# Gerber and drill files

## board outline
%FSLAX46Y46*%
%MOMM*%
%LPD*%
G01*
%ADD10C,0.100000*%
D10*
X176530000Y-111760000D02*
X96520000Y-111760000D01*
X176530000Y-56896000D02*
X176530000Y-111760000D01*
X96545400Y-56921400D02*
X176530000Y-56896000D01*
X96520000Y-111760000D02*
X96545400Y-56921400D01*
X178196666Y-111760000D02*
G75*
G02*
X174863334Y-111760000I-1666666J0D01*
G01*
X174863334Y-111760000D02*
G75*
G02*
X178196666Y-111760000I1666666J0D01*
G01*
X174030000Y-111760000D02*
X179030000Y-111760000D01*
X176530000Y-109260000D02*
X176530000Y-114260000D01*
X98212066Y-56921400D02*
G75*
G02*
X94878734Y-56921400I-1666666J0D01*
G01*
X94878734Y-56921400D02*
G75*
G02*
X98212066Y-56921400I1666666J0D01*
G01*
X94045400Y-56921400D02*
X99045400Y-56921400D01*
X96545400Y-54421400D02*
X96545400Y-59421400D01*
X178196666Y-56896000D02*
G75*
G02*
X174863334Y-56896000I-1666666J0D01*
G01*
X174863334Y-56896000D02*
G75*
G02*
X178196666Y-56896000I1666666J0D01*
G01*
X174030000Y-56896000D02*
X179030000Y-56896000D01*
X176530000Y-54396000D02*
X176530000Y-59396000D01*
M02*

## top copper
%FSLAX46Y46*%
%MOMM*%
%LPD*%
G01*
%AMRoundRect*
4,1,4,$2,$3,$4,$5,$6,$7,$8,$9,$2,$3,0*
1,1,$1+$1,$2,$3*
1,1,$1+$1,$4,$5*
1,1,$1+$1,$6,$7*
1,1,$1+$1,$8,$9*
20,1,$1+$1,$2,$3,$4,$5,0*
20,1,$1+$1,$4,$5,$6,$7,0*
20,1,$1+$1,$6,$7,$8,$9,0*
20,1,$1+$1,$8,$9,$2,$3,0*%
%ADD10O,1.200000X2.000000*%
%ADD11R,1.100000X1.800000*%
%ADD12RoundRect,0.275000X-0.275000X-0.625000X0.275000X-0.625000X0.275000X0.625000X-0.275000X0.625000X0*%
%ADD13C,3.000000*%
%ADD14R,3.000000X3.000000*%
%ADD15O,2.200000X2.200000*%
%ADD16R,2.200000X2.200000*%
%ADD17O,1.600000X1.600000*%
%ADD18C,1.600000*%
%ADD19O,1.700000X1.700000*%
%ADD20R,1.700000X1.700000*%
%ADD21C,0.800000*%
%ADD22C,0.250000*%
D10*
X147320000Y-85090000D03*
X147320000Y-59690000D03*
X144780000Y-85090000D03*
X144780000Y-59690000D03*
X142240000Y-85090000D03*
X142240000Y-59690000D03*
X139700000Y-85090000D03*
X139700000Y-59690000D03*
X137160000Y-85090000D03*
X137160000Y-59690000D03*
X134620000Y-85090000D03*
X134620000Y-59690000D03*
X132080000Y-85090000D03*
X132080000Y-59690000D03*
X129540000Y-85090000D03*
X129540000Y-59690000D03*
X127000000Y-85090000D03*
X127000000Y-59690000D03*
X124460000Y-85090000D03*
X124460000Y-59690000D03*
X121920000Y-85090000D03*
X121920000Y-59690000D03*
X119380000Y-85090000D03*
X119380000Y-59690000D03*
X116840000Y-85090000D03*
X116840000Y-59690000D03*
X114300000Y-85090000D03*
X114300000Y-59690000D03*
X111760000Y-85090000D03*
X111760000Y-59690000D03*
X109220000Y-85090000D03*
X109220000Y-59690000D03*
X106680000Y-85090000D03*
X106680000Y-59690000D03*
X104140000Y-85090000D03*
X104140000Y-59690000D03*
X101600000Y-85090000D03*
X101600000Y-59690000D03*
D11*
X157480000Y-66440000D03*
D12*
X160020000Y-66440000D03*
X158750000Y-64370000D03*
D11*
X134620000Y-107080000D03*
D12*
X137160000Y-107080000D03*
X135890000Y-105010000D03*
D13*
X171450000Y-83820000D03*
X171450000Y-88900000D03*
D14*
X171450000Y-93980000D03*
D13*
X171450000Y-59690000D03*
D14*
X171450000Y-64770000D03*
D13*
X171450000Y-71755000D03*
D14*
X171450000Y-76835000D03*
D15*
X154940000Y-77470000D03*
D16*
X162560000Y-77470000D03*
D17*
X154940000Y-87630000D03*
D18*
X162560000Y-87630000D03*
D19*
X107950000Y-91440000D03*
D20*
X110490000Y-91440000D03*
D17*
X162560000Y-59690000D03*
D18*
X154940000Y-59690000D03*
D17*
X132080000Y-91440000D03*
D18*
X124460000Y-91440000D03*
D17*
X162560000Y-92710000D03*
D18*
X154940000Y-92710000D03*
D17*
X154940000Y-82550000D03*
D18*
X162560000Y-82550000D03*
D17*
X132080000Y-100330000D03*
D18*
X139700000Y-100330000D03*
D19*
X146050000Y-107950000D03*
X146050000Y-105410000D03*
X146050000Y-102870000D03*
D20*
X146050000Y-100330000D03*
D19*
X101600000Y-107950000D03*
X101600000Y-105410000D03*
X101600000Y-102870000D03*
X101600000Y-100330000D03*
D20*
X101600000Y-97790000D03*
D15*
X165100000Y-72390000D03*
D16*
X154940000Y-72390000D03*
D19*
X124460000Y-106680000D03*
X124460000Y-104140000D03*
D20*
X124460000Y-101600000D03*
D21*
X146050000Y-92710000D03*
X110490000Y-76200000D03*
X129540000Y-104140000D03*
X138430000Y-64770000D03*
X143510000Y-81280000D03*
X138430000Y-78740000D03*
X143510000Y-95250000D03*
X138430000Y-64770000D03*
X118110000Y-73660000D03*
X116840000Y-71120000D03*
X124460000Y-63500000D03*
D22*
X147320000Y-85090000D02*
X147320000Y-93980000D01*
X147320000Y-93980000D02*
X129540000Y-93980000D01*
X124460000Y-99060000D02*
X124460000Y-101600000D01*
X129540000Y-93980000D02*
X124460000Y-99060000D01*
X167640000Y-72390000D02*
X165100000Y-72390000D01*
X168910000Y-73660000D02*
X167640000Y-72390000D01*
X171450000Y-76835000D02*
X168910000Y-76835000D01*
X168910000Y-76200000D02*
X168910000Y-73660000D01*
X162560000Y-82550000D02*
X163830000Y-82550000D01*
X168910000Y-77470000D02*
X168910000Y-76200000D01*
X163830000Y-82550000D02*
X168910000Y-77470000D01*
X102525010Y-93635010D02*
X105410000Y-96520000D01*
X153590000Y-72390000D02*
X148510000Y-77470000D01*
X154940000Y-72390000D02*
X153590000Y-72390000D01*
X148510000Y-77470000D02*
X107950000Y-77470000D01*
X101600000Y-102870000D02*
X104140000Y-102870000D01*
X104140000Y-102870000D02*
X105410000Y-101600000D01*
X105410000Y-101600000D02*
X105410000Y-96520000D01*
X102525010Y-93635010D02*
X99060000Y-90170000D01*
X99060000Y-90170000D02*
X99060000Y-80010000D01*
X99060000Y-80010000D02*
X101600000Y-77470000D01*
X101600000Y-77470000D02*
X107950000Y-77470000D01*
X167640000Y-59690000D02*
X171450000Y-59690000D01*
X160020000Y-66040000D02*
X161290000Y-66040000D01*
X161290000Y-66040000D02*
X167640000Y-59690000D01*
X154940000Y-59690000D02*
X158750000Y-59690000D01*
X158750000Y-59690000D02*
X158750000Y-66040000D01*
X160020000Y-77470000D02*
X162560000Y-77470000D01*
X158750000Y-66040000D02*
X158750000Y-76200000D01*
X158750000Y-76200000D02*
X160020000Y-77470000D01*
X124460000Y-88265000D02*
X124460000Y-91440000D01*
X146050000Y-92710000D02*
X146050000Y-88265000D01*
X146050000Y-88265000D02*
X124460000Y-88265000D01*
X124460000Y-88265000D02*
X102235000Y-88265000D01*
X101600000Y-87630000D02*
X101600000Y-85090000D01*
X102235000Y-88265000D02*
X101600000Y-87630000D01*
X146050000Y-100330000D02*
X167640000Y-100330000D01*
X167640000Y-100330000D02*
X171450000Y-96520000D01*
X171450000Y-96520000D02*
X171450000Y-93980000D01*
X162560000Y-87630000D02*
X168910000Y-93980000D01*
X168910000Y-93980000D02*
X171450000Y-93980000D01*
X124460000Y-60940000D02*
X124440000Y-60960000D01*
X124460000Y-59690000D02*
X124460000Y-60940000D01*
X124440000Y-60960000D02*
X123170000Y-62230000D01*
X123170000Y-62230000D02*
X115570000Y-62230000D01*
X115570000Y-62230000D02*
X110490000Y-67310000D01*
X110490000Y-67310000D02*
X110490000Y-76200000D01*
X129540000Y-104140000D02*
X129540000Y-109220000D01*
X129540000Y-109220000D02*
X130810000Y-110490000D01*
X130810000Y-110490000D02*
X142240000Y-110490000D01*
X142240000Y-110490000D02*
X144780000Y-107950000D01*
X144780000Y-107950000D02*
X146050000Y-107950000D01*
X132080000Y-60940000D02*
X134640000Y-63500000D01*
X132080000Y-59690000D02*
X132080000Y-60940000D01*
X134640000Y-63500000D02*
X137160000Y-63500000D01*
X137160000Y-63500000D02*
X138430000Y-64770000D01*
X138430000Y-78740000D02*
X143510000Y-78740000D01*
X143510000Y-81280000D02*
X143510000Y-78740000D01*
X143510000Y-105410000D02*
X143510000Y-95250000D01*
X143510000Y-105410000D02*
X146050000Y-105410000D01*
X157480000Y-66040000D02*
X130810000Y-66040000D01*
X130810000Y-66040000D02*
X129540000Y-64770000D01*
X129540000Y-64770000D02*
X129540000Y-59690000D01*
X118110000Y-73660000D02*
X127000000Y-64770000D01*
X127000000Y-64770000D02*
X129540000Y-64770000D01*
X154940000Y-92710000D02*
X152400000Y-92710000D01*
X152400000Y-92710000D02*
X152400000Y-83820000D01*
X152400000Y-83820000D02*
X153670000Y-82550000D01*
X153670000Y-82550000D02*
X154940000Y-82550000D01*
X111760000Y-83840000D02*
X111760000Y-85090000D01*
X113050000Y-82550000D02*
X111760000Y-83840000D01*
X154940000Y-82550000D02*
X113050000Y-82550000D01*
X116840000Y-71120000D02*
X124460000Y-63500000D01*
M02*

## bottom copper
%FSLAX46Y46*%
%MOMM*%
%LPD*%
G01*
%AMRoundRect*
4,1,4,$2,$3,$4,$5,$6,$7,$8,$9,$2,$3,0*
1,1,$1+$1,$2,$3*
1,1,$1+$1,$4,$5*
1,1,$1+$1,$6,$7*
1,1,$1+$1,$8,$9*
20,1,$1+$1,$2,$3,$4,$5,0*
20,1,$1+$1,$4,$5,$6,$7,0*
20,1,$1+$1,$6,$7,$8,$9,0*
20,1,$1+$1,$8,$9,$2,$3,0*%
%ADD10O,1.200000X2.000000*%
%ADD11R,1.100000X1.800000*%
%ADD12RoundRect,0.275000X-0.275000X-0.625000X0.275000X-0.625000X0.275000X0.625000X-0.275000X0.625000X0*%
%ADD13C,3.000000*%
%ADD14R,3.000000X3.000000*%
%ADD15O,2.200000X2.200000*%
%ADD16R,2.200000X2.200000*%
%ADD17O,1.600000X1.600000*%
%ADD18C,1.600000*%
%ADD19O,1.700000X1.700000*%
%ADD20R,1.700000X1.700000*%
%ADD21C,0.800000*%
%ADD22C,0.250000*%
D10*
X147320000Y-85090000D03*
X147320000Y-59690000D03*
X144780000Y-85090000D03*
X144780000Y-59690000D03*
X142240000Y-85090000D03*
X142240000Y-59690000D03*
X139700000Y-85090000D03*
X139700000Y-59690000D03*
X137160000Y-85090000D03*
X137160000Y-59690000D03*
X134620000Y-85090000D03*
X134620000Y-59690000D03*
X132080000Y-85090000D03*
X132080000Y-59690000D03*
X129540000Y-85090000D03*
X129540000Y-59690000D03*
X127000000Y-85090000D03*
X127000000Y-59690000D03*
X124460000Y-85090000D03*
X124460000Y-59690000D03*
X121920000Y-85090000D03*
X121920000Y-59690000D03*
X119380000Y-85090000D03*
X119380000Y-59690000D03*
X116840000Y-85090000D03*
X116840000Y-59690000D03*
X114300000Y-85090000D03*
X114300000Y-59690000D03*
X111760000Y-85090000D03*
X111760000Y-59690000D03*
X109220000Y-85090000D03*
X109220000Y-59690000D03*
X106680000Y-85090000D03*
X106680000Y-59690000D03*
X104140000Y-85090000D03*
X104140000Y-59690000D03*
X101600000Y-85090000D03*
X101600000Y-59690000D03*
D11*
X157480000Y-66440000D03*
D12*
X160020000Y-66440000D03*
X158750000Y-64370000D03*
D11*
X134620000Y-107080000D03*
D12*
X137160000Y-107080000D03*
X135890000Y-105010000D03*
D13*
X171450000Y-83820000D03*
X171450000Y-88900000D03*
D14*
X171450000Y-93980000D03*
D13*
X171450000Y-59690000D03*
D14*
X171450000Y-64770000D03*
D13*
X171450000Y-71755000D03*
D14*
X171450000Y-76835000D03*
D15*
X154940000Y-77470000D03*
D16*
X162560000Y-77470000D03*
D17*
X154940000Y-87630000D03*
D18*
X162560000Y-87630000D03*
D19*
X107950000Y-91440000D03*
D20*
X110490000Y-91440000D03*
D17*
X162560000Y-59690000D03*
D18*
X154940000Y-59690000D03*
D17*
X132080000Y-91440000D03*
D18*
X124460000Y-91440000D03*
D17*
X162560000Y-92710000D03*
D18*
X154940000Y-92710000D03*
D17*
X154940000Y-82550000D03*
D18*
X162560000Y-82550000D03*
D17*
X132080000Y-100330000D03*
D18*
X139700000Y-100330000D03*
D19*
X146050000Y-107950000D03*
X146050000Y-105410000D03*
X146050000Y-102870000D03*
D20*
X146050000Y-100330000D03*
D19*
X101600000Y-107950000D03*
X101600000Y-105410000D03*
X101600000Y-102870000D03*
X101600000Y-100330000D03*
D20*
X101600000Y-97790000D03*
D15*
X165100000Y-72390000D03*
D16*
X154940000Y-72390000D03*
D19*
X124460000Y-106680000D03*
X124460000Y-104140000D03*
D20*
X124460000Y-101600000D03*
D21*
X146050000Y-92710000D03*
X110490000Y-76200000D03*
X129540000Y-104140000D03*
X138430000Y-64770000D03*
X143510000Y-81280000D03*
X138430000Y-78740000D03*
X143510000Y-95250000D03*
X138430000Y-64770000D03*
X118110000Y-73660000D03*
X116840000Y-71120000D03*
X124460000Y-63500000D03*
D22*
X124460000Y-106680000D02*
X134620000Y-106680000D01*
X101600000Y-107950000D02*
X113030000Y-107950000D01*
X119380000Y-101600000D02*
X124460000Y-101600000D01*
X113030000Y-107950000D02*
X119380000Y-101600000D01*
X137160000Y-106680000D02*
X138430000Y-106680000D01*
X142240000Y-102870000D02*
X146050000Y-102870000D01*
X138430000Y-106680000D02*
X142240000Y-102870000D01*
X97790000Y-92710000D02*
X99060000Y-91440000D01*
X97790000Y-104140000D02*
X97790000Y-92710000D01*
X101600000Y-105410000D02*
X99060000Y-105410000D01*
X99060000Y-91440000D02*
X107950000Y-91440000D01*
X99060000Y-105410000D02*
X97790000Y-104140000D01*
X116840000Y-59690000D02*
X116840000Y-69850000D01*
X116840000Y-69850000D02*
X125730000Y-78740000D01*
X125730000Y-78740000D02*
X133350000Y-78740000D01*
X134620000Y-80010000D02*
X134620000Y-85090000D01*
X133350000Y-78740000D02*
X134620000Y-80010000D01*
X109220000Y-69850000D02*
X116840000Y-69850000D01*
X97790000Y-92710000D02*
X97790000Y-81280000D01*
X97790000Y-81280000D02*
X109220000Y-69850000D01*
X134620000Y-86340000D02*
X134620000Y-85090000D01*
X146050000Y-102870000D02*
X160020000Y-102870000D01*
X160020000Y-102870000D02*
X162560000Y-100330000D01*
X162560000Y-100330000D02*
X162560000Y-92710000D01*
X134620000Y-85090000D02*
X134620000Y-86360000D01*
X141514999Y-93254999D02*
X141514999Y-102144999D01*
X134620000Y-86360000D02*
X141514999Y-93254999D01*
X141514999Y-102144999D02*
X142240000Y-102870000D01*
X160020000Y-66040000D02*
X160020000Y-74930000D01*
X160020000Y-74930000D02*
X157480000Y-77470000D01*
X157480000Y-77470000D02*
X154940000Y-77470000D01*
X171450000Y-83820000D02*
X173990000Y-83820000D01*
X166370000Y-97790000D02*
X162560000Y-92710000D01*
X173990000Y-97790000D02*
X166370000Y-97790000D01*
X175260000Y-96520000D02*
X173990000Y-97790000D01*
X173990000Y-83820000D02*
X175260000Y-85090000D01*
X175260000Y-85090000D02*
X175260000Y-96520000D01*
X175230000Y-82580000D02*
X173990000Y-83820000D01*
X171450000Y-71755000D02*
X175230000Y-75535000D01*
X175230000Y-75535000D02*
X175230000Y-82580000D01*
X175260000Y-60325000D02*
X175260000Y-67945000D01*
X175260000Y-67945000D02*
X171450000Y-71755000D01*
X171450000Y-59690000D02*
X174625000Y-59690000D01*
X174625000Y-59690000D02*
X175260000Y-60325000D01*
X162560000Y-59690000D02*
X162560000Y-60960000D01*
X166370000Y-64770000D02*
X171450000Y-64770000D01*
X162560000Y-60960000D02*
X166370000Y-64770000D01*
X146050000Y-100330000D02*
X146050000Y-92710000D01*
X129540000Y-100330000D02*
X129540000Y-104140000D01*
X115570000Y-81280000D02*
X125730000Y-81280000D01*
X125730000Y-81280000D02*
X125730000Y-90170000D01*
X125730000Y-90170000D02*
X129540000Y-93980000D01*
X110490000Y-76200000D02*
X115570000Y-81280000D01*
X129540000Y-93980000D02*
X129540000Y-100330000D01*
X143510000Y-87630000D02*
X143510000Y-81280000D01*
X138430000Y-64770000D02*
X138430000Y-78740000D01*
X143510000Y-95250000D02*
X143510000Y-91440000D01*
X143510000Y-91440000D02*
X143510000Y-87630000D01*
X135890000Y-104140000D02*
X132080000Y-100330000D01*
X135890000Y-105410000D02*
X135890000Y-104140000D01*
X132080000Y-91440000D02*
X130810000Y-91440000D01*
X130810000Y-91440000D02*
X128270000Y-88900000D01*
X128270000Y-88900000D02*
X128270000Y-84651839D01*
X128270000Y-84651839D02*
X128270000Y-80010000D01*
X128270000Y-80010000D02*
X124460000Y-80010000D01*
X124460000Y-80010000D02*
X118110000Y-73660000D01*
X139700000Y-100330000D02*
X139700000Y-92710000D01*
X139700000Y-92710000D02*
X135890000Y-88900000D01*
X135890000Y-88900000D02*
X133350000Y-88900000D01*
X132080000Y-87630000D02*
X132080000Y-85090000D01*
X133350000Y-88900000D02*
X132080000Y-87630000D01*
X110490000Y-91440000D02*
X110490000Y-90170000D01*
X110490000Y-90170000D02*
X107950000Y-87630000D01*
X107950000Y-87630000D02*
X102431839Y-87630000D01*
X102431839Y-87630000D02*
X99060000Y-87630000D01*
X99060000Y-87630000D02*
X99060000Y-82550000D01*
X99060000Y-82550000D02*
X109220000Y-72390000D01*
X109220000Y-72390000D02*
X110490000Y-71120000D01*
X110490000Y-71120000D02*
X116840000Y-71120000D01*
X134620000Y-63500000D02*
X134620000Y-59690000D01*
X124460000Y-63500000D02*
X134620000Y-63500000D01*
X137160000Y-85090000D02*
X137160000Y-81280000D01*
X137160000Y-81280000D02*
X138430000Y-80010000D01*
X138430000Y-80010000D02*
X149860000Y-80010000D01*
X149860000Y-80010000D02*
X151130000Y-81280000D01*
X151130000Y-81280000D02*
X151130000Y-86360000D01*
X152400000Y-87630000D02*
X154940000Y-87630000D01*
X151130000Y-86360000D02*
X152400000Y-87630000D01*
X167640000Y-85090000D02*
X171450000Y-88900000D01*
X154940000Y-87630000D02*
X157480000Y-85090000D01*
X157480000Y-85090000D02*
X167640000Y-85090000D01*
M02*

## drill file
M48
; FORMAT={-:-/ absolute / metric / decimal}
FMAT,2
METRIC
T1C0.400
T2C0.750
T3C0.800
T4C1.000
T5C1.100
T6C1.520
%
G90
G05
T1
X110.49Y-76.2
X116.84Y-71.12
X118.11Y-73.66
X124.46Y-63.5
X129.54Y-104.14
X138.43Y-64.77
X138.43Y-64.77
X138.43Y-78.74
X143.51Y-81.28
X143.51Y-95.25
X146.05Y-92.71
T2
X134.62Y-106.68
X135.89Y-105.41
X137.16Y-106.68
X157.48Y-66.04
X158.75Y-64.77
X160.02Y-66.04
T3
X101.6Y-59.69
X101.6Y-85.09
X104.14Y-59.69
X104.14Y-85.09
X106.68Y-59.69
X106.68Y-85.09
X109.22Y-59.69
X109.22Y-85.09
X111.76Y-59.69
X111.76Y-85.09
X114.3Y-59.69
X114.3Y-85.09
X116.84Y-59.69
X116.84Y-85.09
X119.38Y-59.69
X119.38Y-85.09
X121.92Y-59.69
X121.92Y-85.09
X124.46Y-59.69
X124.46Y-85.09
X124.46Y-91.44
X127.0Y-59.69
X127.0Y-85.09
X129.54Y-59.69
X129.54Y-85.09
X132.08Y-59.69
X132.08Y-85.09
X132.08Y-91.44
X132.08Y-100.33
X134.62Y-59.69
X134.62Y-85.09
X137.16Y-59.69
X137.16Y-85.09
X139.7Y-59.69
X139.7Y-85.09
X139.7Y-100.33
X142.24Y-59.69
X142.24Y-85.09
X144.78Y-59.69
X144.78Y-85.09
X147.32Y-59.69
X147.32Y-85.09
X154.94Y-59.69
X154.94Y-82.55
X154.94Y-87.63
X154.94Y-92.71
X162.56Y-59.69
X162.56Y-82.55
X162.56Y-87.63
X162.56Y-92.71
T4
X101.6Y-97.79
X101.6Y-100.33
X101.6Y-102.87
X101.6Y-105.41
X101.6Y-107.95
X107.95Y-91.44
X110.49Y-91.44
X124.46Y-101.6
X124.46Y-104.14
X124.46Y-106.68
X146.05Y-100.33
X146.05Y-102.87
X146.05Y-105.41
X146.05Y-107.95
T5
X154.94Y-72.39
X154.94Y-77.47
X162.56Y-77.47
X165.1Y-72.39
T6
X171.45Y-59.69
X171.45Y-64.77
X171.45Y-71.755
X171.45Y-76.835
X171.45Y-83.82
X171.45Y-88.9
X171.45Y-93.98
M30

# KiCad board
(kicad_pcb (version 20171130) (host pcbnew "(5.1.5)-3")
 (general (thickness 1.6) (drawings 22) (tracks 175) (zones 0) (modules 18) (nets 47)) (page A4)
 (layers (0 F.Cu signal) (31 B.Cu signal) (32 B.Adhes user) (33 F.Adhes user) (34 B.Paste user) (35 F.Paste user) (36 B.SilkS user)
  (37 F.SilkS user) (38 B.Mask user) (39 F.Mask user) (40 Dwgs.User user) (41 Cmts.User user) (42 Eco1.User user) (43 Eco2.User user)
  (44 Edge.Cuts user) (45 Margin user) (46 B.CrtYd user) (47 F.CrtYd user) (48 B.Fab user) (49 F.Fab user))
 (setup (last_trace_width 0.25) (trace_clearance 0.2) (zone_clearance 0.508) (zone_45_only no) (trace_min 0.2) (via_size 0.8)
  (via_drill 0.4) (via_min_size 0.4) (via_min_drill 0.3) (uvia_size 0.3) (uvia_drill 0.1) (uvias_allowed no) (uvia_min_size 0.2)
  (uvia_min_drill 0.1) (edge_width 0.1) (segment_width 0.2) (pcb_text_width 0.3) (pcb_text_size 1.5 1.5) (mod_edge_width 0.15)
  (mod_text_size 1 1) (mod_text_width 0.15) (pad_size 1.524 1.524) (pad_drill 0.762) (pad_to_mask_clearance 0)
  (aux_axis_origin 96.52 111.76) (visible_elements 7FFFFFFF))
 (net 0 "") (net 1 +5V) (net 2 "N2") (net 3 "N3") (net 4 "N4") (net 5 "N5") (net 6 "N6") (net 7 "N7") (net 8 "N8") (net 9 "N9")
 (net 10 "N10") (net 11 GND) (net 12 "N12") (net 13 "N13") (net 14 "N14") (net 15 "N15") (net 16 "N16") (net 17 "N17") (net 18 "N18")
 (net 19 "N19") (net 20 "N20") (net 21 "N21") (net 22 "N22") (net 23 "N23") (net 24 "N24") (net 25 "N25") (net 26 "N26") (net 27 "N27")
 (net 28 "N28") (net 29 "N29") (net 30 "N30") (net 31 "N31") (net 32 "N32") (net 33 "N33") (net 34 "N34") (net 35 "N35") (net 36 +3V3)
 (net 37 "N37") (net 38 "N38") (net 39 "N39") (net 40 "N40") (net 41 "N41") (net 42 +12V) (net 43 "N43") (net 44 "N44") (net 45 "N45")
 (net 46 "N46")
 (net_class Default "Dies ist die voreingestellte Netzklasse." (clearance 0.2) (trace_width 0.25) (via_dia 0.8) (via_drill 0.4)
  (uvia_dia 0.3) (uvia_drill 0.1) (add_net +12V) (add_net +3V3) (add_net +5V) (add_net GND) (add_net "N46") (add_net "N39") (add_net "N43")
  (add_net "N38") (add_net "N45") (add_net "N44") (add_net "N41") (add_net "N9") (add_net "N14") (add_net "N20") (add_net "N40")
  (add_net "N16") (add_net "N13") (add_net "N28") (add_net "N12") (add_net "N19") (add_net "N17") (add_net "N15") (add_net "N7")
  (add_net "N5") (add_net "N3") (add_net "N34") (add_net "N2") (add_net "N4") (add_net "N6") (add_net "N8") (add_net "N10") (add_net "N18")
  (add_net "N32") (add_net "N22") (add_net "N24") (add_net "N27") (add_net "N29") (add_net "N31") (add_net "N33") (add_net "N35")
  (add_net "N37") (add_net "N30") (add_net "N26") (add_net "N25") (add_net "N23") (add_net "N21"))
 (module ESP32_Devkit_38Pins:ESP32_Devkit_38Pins (layer F.Cu) (at 124.46 72.39)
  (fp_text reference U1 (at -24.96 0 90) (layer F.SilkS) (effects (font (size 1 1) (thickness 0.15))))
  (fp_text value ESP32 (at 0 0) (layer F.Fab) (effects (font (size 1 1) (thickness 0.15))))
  (pad 19 thru_hole oval (at 22.86 12.7) (size 1.2 2) (drill 0.8) (layers *.Cu *.Mask) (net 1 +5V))
  (pad 20 thru_hole oval (at 22.86 -12.7) (size 1.2 2) (drill 0.8) (layers *.Cu *.Mask) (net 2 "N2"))
  (pad 18 thru_hole oval (at 20.32 12.7) (size 1.2 2) (drill 0.8) (layers *.Cu *.Mask) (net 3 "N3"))
  (pad 21 thru_hole oval (at 20.32 -12.7) (size 1.2 2) (drill 0.8) (layers *.Cu *.Mask) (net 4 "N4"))
  (pad 17 thru_hole oval (at 17.78 12.7) (size 1.2 2) (drill 0.8) (layers *.Cu *.Mask) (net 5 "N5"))
  (pad 22 thru_hole oval (at 17.78 -12.7) (size 1.2 2) (drill 0.8) (layers *.Cu *.Mask) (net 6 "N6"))
  (pad 16 thru_hole oval (at 15.24 12.7) (size 1.2 2) (drill 0.8) (layers *.Cu *.Mask) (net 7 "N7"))
  (pad 23 thru_hole oval (at 15.24 -12.7) (size 1.2 2) (drill 0.8) (layers *.Cu *.Mask) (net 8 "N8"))
  (pad 15 thru_hole oval (at 12.7 12.7) (size 1.2 2) (drill 0.8) (layers *.Cu *.Mask) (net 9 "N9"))
  (pad 24 thru_hole oval (at 12.7 -12.7) (size 1.2 2) (drill 0.8) (layers *.Cu *.Mask) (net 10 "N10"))
  (pad 14 thru_hole oval (at 10.16 12.7) (size 1.2 2) (drill 0.8) (layers *.Cu *.Mask) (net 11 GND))
  (pad 25 thru_hole oval (at 10.16 -12.7) (size 1.2 2) (drill 0.8) (layers *.Cu *.Mask) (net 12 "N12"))
  (pad 13 thru_hole oval (at 7.62 12.7) (size 1.2 2) (drill 0.8) (layers *.Cu *.Mask) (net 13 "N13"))
  (pad 26 thru_hole oval (at 7.62 -12.7) (size 1.2 2) (drill 0.8) (layers *.Cu *.Mask) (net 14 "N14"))
  (pad 12 thru_hole oval (at 5.08 12.7) (size 1.2 2) (drill 0.8) (layers *.Cu *.Mask) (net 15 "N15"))
  (pad 27 thru_hole oval (at 5.08 -12.7) (size 1.2 2) (drill 0.8) (layers *.Cu *.Mask) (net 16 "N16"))
  (pad 11 thru_hole oval (at 2.54 12.7) (size 1.2 2) (drill 0.8) (layers *.Cu *.Mask) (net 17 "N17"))
  (pad 28 thru_hole oval (at 2.54 -12.7) (size 1.2 2) (drill 0.8) (layers *.Cu *.Mask) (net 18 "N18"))
  (pad 10 thru_hole oval (at 0 12.7) (size 1.2 2) (drill 0.8) (layers *.Cu *.Mask) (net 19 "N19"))
  (pad 29 thru_hole oval (at 0 -12.7) (size 1.2 2) (drill 0.8) (layers *.Cu *.Mask) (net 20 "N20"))
  (pad 9 thru_hole oval (at -2.54 12.7) (size 1.2 2) (drill 0.8) (layers *.Cu *.Mask) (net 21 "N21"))
  (pad 30 thru_hole oval (at -2.54 -12.7) (size 1.2 2) (drill 0.8) (layers *.Cu *.Mask) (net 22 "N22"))
  (pad 8 thru_hole oval (at -5.08 12.7) (size 1.2 2) (drill 0.8) (layers *.Cu *.Mask) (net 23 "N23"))
  (pad 31 thru_hole oval (at -5.08 -12.7) (size 1.2 2) (drill 0.8) (layers *.Cu *.Mask) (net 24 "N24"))
  (pad 7 thru_hole oval (at -7.62 12.7) (size 1.2 2) (drill 0.8) (layers *.Cu *.Mask) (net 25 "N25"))
  (pad 32 thru_hole oval (at -7.62 -12.7) (size 1.2 2) (drill 0.8) (layers *.Cu *.Mask) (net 11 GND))
  (pad 6 thru_hole oval (at -10.16 12.7) (size 1.2 2) (drill 0.8) (layers *.Cu *.Mask) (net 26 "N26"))
  (pad 33 thru_hole oval (at -10.16 -12.7) (size 1.2 2) (drill 0.8) (layers *.Cu *.Mask) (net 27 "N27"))
  (pad 5 thru_hole oval (at -12.7 12.7) (size 1.2 2) (drill 0.8) (layers *.Cu *.Mask) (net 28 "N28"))
  (pad 34 thru_hole oval (at -12.7 -12.7) (size 1.2 2) (drill 0.8) (layers *.Cu *.Mask) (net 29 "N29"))
  (pad 4 thru_hole oval (at -15.24 12.7) (size 1.2 2) (drill 0.8) (layers *.Cu *.Mask) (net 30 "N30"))
  (pad 35 thru_hole oval (at -15.24 -12.7) (size 1.2 2) (drill 0.8) (layers *.Cu *.Mask) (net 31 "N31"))
  (pad 3 thru_hole oval (at -17.78 12.7) (size 1.2 2) (drill 0.8) (layers *.Cu *.Mask) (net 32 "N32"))
  (pad 36 thru_hole oval (at -17.78 -12.7) (size 1.2 2) (drill 0.8) (layers *.Cu *.Mask) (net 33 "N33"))
  (pad 2 thru_hole oval (at -20.32 12.7) (size 1.2 2) (drill 0.8) (layers *.Cu *.Mask) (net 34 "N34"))
  (pad 37 thru_hole oval (at -20.32 -12.7) (size 1.2 2) (drill 0.8) (layers *.Cu *.Mask) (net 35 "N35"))
  (pad 1 thru_hole oval (at -22.86 12.7) (size 1.2 2) (drill 0.8) (layers *.Cu *.Mask) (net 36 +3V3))
  (pad 38 thru_hole oval (at -22.86 -12.7) (size 1.2 2) (drill 0.8) (layers *.Cu *.Mask) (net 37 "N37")))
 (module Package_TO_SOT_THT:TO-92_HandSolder (layer F.Cu) (at 157.48 66.04)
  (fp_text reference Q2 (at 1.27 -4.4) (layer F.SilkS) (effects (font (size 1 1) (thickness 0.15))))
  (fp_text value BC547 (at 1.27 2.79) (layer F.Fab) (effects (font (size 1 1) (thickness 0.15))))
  (pad 1 thru_hole rect (at 0 0) (size 1.1 1.8) (drill 0.75 (offset 0 0.4)) (layers *.Cu *.Mask) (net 16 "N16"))
  (pad 3 thru_hole roundrect (at 2.54 0) (size 1.1 1.8) (drill 0.75 (offset 0 0.4)) (layers *.Cu *.Mask) (roundrect_rratio 0.25)
   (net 11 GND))
  (pad 2 thru_hole roundrect (at 1.27 -1.27) (size 1.1 1.8) (drill 0.75 (offset 0 -0.4)) (layers *.Cu *.Mask) (roundrect_rratio 0.25)
   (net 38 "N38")))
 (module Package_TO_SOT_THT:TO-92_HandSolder (layer F.Cu) (at 134.62 106.68)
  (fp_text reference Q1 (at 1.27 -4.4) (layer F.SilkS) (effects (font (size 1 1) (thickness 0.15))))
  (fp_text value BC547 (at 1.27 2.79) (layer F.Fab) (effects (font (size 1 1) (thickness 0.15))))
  (pad 1 thru_hole rect (at 0 0) (size 1.1 1.8) (drill 0.75 (offset 0 0.4)) (layers *.Cu *.Mask) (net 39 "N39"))
  (pad 3 thru_hole roundrect (at 2.54 0) (size 1.1 1.8) (drill 0.75 (offset 0 0.4)) (layers *.Cu *.Mask) (roundrect_rratio 0.25)
   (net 11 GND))
  (pad 2 thru_hole roundrect (at 1.27 -1.27) (size 1.1 1.8) (drill 0.75 (offset 0 -0.4)) (layers *.Cu *.Mask) (roundrect_rratio 0.25)
   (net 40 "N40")))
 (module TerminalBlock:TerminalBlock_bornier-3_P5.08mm (layer F.Cu) (at 171.45 93.98 90)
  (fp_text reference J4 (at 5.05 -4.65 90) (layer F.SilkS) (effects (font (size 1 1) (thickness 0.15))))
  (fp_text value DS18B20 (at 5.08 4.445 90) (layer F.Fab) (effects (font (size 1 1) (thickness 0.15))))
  (pad 3 thru_hole circle (at 10.16 0 90) (size 3 3) (drill 1.52) (layers *.Cu *.Mask) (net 11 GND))
  (pad 2 thru_hole circle (at 5.08 0 90) (size 3 3) (drill 1.52) (layers *.Cu *.Mask) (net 9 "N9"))
  (pad 1 thru_hole rect (at 0 0 90) (size 3 3) (drill 1.52) (layers *.Cu *.Mask) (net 36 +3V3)))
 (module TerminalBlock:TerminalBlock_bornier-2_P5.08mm (layer F.Cu) (at 171.45 64.77 90)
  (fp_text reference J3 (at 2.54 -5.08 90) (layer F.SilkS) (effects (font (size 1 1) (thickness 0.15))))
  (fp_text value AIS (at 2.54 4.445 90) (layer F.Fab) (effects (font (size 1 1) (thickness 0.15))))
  (pad 2 thru_hole circle (at 5.08 0 90) (size 3 3) (drill 1.52) (layers *.Cu *.Mask) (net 11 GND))
  (pad 1 thru_hole rect (at 0 0 90) (size 3 3) (drill 1.52) (layers *.Cu *.Mask) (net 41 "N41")))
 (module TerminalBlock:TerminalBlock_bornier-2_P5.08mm (layer F.Cu) (at 171.45 76.835 90)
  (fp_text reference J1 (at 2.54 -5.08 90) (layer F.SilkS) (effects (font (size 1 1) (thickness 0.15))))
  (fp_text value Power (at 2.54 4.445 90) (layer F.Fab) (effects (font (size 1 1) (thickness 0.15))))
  (pad 2 thru_hole circle (at 5.08 0 90) (size 3 3) (drill 1.52) (layers *.Cu *.Mask) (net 11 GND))
  (pad 1 thru_hole rect (at 0 0 90) (size 3 3) (drill 1.52) (layers *.Cu *.Mask) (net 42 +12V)))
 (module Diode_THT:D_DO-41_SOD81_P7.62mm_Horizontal (layer F.Cu) (at 162.56 77.47 180)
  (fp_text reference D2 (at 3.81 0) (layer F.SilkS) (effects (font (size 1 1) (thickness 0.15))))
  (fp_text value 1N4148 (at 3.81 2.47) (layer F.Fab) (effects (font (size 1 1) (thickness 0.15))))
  (pad 2 thru_hole oval (at 7.62 0 180) (size 2.2 2.2) (drill 1.1) (layers *.Cu *.Mask) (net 11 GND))
  (pad 1 thru_hole rect (at 0 0 180) (size 2.2 2.2) (drill 1.1) (layers *.Cu *.Mask) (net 38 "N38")))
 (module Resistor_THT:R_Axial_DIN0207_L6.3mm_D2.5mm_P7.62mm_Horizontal (layer F.Cu) (at 162.56 87.63 180)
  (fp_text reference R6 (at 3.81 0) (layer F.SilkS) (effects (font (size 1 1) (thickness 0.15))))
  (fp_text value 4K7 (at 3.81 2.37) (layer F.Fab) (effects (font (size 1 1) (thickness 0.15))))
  (pad 2 thru_hole oval (at 7.62 0 180) (size 1.6 1.6) (drill 0.8) (layers *.Cu *.Mask) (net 9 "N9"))
  (pad 1 thru_hole circle (at 0 0 180) (size 1.6 1.6) (drill 0.8) (layers *.Cu *.Mask) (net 36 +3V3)))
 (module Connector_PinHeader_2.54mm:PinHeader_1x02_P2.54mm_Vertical (layer F.Cu) (at 110.49 91.44 270)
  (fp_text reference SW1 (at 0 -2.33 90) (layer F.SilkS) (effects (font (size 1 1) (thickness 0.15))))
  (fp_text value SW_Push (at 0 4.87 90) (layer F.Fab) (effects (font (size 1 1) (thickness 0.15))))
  (pad 2 thru_hole oval (at 0 2.54 270) (size 1.7 1.7) (drill 1) (layers *.Cu *.Mask) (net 11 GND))
  (pad 1 thru_hole rect (at 0 0 270) (size 1.7 1.7) (drill 1) (layers *.Cu *.Mask) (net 12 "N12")))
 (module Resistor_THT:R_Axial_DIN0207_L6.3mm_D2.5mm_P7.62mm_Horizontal (layer F.Cu) (at 154.94 59.69)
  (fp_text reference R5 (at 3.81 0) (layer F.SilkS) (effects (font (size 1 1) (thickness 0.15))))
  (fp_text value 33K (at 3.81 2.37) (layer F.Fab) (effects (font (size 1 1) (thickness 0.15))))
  (pad 2 thru_hole oval (at 7.62 0) (size 1.6 1.6) (drill 0.8) (layers *.Cu *.Mask) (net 41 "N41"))
  (pad 1 thru_hole circle (at 0 0) (size 1.6 1.6) (drill 0.8) (layers *.Cu *.Mask) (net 38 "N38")))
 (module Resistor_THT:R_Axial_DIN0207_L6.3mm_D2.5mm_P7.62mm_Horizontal (layer F.Cu) (at 124.46 91.44)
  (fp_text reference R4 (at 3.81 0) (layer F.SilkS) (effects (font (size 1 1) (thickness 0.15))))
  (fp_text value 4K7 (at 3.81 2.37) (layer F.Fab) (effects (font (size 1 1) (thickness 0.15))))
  (pad 2 thru_hole oval (at 7.62 0) (size 1.6 1.6) (drill 0.8) (layers *.Cu *.Mask) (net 16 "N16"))
  (pad 1 thru_hole circle (at 0 0) (size 1.6 1.6) (drill 0.8) (layers *.Cu *.Mask) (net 36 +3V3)))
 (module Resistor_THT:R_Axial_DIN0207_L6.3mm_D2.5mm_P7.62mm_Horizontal (layer F.Cu) (at 154.94 92.71)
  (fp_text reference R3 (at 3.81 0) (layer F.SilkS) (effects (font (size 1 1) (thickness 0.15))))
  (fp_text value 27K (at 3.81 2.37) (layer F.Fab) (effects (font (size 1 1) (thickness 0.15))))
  (pad 2 thru_hole oval (at 7.62 0) (size 1.6 1.6) (drill 0.8) (layers *.Cu *.Mask) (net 11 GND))
  (pad 1 thru_hole circle (at 0 0) (size 1.6 1.6) (drill 0.8) (layers *.Cu *.Mask) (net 28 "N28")))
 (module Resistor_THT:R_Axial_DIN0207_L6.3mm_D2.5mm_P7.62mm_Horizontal (layer F.Cu) (at 162.56 82.55 180)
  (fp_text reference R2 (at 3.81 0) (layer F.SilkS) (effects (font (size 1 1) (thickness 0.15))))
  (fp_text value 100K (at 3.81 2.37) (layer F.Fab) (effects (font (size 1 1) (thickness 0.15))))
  (pad 2 thru_hole oval (at 7.62 0 180) (size 1.6 1.6) (drill 0.8) (layers *.Cu *.Mask) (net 28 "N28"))
  (pad 1 thru_hole circle (at 0 0 180) (size 1.6 1.6) (drill 0.8) (layers *.Cu *.Mask) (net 42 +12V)))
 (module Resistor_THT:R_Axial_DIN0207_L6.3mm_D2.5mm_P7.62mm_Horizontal (layer F.Cu) (at 139.7 100.33 180)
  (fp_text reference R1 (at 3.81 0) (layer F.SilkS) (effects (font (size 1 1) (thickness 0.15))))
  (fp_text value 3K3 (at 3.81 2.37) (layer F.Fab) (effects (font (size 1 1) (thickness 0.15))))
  (pad 2 thru_hole oval (at 7.62 0 180) (size 1.6 1.6) (drill 0.8) (layers *.Cu *.Mask) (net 40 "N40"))
  (pad 1 thru_hole circle (at 0 0 180) (size 1.6 1.6) (drill 0.8) (layers *.Cu *.Mask) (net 13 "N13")))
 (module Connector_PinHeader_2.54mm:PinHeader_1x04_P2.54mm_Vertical (layer F.Cu) (at 146.05 100.33)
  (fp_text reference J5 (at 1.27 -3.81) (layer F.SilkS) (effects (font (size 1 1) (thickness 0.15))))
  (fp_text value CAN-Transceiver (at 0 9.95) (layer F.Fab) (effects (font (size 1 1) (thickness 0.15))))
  (pad 4 thru_hole oval (at 0 7.62) (size 1.7 1.7) (drill 1) (layers *.Cu *.Mask) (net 20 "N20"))
  (pad 3 thru_hole oval (at 0 5.08) (size 1.7 1.7) (drill 1) (layers *.Cu *.Mask) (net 14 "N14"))
  (pad 2 thru_hole oval (at 0 2.54) (size 1.7 1.7) (drill 1) (layers *.Cu *.Mask) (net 11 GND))
  (pad 1 thru_hole rect (at 0 0) (size 1.7 1.7) (drill 1) (layers *.Cu *.Mask) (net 36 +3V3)))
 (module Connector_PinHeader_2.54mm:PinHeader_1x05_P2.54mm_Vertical (layer F.Cu) (at 101.6 97.79)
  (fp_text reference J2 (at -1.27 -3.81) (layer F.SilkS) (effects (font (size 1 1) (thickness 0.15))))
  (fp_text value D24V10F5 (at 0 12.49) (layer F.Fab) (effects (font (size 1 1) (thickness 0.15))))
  (pad 5 thru_hole oval (at 0 10.16) (size 1.7 1.7) (drill 1) (layers *.Cu *.Mask) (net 1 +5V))
  (pad 4 thru_hole oval (at 0 7.62) (size 1.7 1.7) (drill 1) (layers *.Cu *.Mask) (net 11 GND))
  (pad 3 thru_hole oval (at 0 5.08) (size 1.7 1.7) (drill 1) (layers *.Cu *.Mask) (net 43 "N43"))
  (pad 2 thru_hole oval (at 0 2.54) (size 1.7 1.7) (drill 1) (layers *.Cu *.Mask) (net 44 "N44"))
  (pad 1 thru_hole rect (at 0 0) (size 1.7 1.7) (drill 1) (layers *.Cu *.Mask) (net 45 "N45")))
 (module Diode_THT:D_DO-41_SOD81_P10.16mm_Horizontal (layer F.Cu) (at 154.94 72.39)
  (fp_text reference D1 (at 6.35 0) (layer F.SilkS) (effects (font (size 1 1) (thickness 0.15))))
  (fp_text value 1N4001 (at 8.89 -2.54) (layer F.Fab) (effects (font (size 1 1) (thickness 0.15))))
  (pad 2 thru_hole oval (at 10.16 0) (size 2.2 2.2) (drill 1.1) (layers *.Cu *.Mask) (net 42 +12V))
  (pad 1 thru_hole rect (at 0 0) (size 2.2 2.2) (drill 1.1) (layers *.Cu *.Mask) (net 43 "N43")))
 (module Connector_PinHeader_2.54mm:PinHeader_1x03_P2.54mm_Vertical (layer F.Cu) (at 124.46 101.6)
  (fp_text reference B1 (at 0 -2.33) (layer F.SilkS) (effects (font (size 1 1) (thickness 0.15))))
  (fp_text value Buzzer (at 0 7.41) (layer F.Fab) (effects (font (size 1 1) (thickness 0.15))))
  (pad 3 thru_hole oval (at 0 5.08) (size 1.7 1.7) (drill 1) (layers *.Cu *.Mask) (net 39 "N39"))
  (pad 2 thru_hole oval (at 0 2.54) (size 1.7 1.7) (drill 1) (layers *.Cu *.Mask) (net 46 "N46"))
  (pad 1 thru_hole rect (at 0 0) (size 1.7 1.7) (drill 1) (layers *.Cu *.Mask) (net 1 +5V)))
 (gr_line (start 176.53 111.76) (end 96.52 111.76) (layer Edge.Cuts) (width 0.1))
 (gr_line (start 176.53 56.896) (end 176.53 111.76) (layer Edge.Cuts) (width 0.1))
 (gr_line (start 96.5454 56.9214) (end 176.53 56.896) (layer Edge.Cuts) (width 0.1))
 (gr_line (start 96.52 111.76) (end 96.5454 56.9214) (layer Edge.Cuts) (width 0.1))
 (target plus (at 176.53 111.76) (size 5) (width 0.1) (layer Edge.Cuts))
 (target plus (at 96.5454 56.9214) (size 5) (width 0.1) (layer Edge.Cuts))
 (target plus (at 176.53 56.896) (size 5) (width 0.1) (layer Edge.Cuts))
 (segment (start 124.46 106.68) (end 134.62 106.68) (width 0.25) (layer B.Cu) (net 39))
 (segment (start 101.6 107.95) (end 113.03 107.95) (width 0.25) (layer B.Cu) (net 1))
 (segment (start 119.38 101.6) (end 124.46 101.6) (width 0.25) (layer B.Cu) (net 1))
 (segment (start 113.03 107.95) (end 119.38 101.6) (width 0.25) (layer B.Cu) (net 1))
 (segment (start 147.32 85.09) (end 147.32 93.98) (width 0.25) (layer F.Cu) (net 1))
 (segment (start 147.32 93.98) (end 129.54 93.98) (width 0.25) (layer F.Cu) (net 1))
 (segment (start 124.46 99.06) (end 124.46 101.6) (width 0.25) (layer F.Cu) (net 1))
 (segment (start 129.54 93.98) (end 124.46 99.06) (width 0.25) (layer F.Cu) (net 1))
 (segment (start 167.64 72.39) (end 165.1 72.39) (width 0.25) (layer F.Cu) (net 42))
 (segment (start 168.91 73.66) (end 167.64 72.39) (width 0.25) (layer F.Cu) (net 42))
 (segment (start 171.45 76.835) (end 168.91 76.835) (width 0.25) (layer F.Cu) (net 42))
 (segment (start 168.91 76.2) (end 168.91 73.66) (width 0.25) (layer F.Cu) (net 42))
 (segment (start 162.56 82.55) (end 163.83 82.55) (width 0.25) (layer F.Cu) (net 42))
 (segment (start 168.91 77.47) (end 168.91 76.2) (width 0.25) (layer F.Cu) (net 42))
 (segment (start 163.83 82.55) (end 168.91 77.47) (width 0.25) (layer F.Cu) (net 42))
 (segment (start 102.52501 93.63501) (end 105.41 96.52) (width 0.25) (layer F.Cu) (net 43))
 (segment (start 153.59 72.39) (end 148.51 77.47) (width 0.25) (layer F.Cu) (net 43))
 (segment (start 154.94 72.39) (end 153.59 72.39) (width 0.25) (layer F.Cu) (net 43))
 (segment (start 148.51 77.47) (end 107.95 77.47) (width 0.25) (layer F.Cu) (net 43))
 (segment (start 101.6 102.87) (end 104.14 102.87) (width 0.25) (layer F.Cu) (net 43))
 (segment (start 104.14 102.87) (end 105.41 101.6) (width 0.25) (layer F.Cu) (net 43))
 (segment (start 105.41 101.6) (end 105.41 96.52) (width 0.25) (layer F.Cu) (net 43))
 (segment (start 102.52501 93.63501) (end 99.06 90.17) (width 0.25) (layer F.Cu) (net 43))
 (segment (start 99.06 90.17) (end 99.06 80.01) (width 0.25) (layer F.Cu) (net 43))
 (segment (start 99.06 80.01) (end 101.6 77.47) (width 0.25) (layer F.Cu) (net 43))
 (segment (start 101.6 77.47) (end 107.95 77.47) (width 0.25) (layer F.Cu) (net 43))
 (segment (start 137.16 106.68) (end 138.43 106.68) (width 0.25) (layer B.Cu) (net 11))
 (segment (start 142.24 102.87) (end 146.05 102.87) (width 0.25) (layer B.Cu) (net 11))
 (segment (start 138.43 106.68) (end 142.24 102.87) (width 0.25) (layer B.Cu) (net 11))
 (segment (start 97.79 92.71) (end 99.06 91.44) (width 0.25) (layer B.Cu) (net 11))
 (segment (start 97.79 104.14) (end 97.79 92.71) (width 0.25) (layer B.Cu) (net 11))
 (segment (start 101.6 105.41) (end 99.06 105.41) (width 0.25) (layer B.Cu) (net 11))
 (segment (start 99.06 91.44) (end 107.95 91.44) (width 0.25) (layer B.Cu) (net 11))
 (segment (start 99.06 105.41) (end 97.79 104.14) (width 0.25) (layer B.Cu) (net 11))
 (segment (start 116.84 59.69) (end 116.84 69.85) (width 0.25) (layer B.Cu) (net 11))
 (segment (start 116.84 69.85) (end 125.73 78.74) (width 0.25) (layer B.Cu) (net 11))
 (segment (start 125.73 78.74) (end 133.35 78.74) (width 0.25) (layer B.Cu) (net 11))
 (segment (start 134.62 80.01) (end 134.62 85.09) (width 0.25) (layer B.Cu) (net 11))
 (segment (start 133.35 78.74) (end 134.62 80.01) (width 0.25) (layer B.Cu) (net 11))
 (segment (start 109.22 69.85) (end 116.84 69.85) (width 0.25) (layer B.Cu) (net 11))
 (segment (start 97.79 92.71) (end 97.79 81.28) (width 0.25) (layer B.Cu) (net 11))
 (segment (start 97.79 81.28) (end 109.22 69.85) (width 0.25) (layer B.Cu) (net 11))
 (segment (start 134.62 86.34) (end 134.62 85.09) (width 0.25) (layer B.Cu) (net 11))
 (segment (start 146.05 102.87) (end 160.02 102.87) (width 0.25) (layer B.Cu) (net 11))
 (segment (start 160.02 102.87) (end 162.56 100.33) (width 0.25) (layer B.Cu) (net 11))
 (segment (start 162.56 100.33) (end 162.56 92.71) (width 0.25) (layer B.Cu) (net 11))
 (segment (start 134.62 85.09) (end 134.62 86.36) (width 0.25) (layer B.Cu) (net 11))
 (segment (start 141.514999 93.254999) (end 141.514999 102.144999) (width 0.25) (layer B.Cu) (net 11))
 (segment (start 134.62 86.36) (end 141.514999 93.254999) (width 0.25) (layer B.Cu) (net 11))
 (segment (start 141.514999 102.144999) (end 142.24 102.87) (width 0.25) (layer B.Cu) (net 11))
 (segment (start 160.02 66.04) (end 160.02 74.93) (width 0.25) (layer B.Cu) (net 11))
 (segment (start 160.02 74.93) (end 157.48 77.47) (width 0.25) (layer B.Cu) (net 11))
 (segment (start 157.48 77.47) (end 154.94 77.47) (width 0.25) (layer B.Cu) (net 11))
 (segment (start 171.45 83.82) (end 173.99 83.82) (width 0.25) (layer B.Cu) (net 11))
 (segment (start 166.37 97.79) (end 162.56 92.71) (width 0.25) (layer B.Cu) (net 11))
 (segment (start 173.99 97.79) (end 166.37 97.79) (width 0.25) (layer B.Cu) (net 11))
 (segment (start 175.26 96.52) (end 173.99 97.79) (width 0.25) (layer B.Cu) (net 11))
 (segment (start 173.99 83.82) (end 175.26 85.09) (width 0.25) (layer B.Cu) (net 11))
 (segment (start 175.26 85.09) (end 175.26 96.52) (width 0.25) (layer B.Cu) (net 11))
 (segment (start 175.23 82.58) (end 173.99 83.82) (width 0.25) (layer B.Cu) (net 11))
 (segment (start 171.45 71.755) (end 175.23 75.535) (width 0.25) (layer B.Cu) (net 11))
 (segment (start 175.23 75.535) (end 175.23 82.58) (width 0.25) (layer B.Cu) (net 11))
 (segment (start 167.64 59.69) (end 171.45 59.69) (width 0.25) (layer F.Cu) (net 11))
 (segment (start 160.02 66.04) (end 161.29 66.04) (width 0.25) (layer F.Cu) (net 11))
 (segment (start 161.29 66.04) (end 167.64 59.69) (width 0.25) (layer F.Cu) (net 11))
 (segment (start 175.26 60.325) (end 175.26 67.945) (width 0.25) (layer B.Cu) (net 11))
 (segment (start 175.26 67.945) (end 171.45 71.755) (width 0.25) (layer B.Cu) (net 11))
 (segment (start 171.45 59.69) (end 174.625 59.69) (width 0.25) (layer B.Cu) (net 11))
 (segment (start 174.625 59.69) (end 175.26 60.325) (width 0.25) (layer B.Cu) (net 11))
 (segment (start 154.94 59.69) (end 158.75 59.69) (width 0.25) (layer F.Cu) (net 38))
 (segment (start 158.75 59.69) (end 158.75 66.04) (width 0.25) (layer F.Cu) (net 38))
 (segment (start 160.02 77.47) (end 162.56 77.47) (width 0.25) (layer F.Cu) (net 38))
 (segment (start 158.75 66.04) (end 158.75 76.2) (width 0.25) (layer F.Cu) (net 38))
 (segment (start 158.75 76.2) (end 160.02 77.47) (width 0.25) (layer F.Cu) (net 38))
 (segment (start 162.56 59.69) (end 162.56 60.96) (width 0.25) (layer B.Cu) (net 41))
 (segment (start 166.37 64.77) (end 171.45 64.77) (width 0.25) (layer B.Cu) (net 41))
 (segment (start 162.56 60.96) (end 166.37 64.77) (width 0.25) (layer B.Cu) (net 41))
 (segment (start 146.05 100.33) (end 146.05 92.71) (width 0.25) (layer B.Cu) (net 36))
 (via (at 146.05 92.71) (size 0.8) (drill 0.4) (layers F.Cu B.Cu) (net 36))
 (segment (start 124.46 88.265) (end 124.46 91.44) (width 0.25) (layer F.Cu) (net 36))
 (segment (start 146.05 92.71) (end 146.05 88.265) (width 0.25) (layer F.Cu) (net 36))
 (segment (start 146.05 88.265) (end 124.46 88.265) (width 0.25) (layer F.Cu) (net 36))
 (segment (start 124.46 88.265) (end 102.235 88.265) (width 0.25) (layer F.Cu) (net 36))
 (segment (start 101.6 87.63) (end 101.6 85.09) (width 0.25) (layer F.Cu) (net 36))
 (segment (start 102.235 88.265) (end 101.6 87.63) (width 0.25) (layer F.Cu) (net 36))
 (segment (start 146.05 100.33) (end 167.64 100.33) (width 0.25) (layer F.Cu) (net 36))
 (segment (start 167.64 100.33) (end 171.45 96.52) (width 0.25) (layer F.Cu) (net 36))
 (segment (start 171.45 96.52) (end 171.45 93.98) (width 0.25) (layer F.Cu) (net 36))
 (segment (start 162.56 87.63) (end 168.91 93.98) (width 0.25) (layer F.Cu) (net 36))
 (segment (start 168.91 93.98) (end 171.45 93.98) (width 0.25) (layer F.Cu) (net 36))
 (segment (start 124.46 60.94) (end 124.44 60.96) (width 0.25) (layer F.Cu) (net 20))
 (segment (start 124.46 59.69) (end 124.46 60.94) (width 0.25) (layer F.Cu) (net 20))
 (segment (start 124.44 60.96) (end 123.17 62.23) (width 0.25) (layer F.Cu) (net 20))
 (segment (start 123.17 62.23) (end 115.57 62.23) (width 0.25) (layer F.Cu) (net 20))
 (segment (start 115.57 62.23) (end 110.49 67.31) (width 0.25) (layer F.Cu) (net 20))
 (via (at 110.49 76.2) (size 0.8) (drill 0.4) (layers F.Cu B.Cu) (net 20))
 (segment (start 110.49 67.31) (end 110.49 76.2) (width 0.25) (layer F.Cu) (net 20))
 (via (at 129.54 104.14) (size 0.8) (drill 0.4) (layers F.Cu B.Cu) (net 20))
 (segment (start 129.54 104.14) (end 129.54 109.22) (width 0.25) (layer F.Cu) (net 20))
 (segment (start 129.54 109.22) (end 130.81 110.49) (width 0.25) (layer F.Cu) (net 20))
 (segment (start 130.81 110.49) (end 142.24 110.49) (width 0.25) (layer F.Cu) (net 20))
 (segment (start 142.24 110.49) (end 144.78 107.95) (width 0.25) (layer F.Cu) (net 20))
 (segment (start 144.78 107.95) (end 146.05 107.95) (width 0.25) (layer F.Cu) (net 20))
 (segment (start 129.54 100.33) (end 129.54 104.14) (width 0.25) (layer B.Cu) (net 20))
 (segment (start 115.57 81.28) (end 125.73 81.28) (width 0.25) (layer B.Cu) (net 20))
 (segment (start 125.73 81.28) (end 125.73 90.17) (width 0.25) (layer B.Cu) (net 20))
 (segment (start 125.73 90.17) (end 129.54 93.98) (width 0.25) (layer B.Cu) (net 20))
 (segment (start 110.49 76.2) (end 115.57 81.28) (width 0.25) (layer B.Cu) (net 20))
 (segment (start 129.54 93.98) (end 129.54 100.33) (width 0.25) (layer B.Cu) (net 20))
 (segment (start 132.08 60.94) (end 134.64 63.5) (width 0.25) (layer F.Cu) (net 14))
 (segment (start 132.08 59.69) (end 132.08 60.94) (width 0.25) (layer F.Cu) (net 14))
 (segment (start 134.64 63.5) (end 137.16 63.5) (width 0.25) (layer F.Cu) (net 14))
 (segment (start 137.16 63.5) (end 138.43 64.77) (width 0.25) (layer F.Cu) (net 14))
 (via (at 138.43 64.77) (size 0.8) (drill 0.4) (layers F.Cu B.Cu) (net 14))
 (via (at 143.51 81.28) (size 0.8) (drill 0.4) (layers F.Cu B.Cu) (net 14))
 (via (at 138.43 78.74) (size 0.8) (drill 0.4) (layers F.Cu B.Cu) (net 14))
 (via (at 143.51 95.25) (size 0.8) (drill 0.4) (layers F.Cu B.Cu) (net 14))
 (via (at 138.43 64.77) (size 0.8) (drill 0.4) (layers F.Cu B.Cu) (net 14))
 (segment (start 138.43 78.74) (end 143.51 78.74) (width 0.25) (layer F.Cu) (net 14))
 (segment (start 143.51 87.63) (end 143.51 81.28) (width 0.25) (layer B.Cu) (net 14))
 (segment (start 143.51 81.28) (end 143.51 78.74) (width 0.25) (layer F.Cu) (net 14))
 (segment (start 138.43 64.77) (end 138.43 78.74) (width 0.25) (layer B.Cu) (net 14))
 (segment (start 143.51 105.41) (end 143.51 95.25) (width 0.25) (layer F.Cu) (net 14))
 (segment (start 143.51 95.25) (end 143.51 91.44) (width 0.25) (layer B.Cu) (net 14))
 (segment (start 143.51 91.44) (end 143.51 87.63) (width 0.25) (layer B.Cu) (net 14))
 (segment (start 143.51 105.41) (end 146.05 105.41) (width 0.25) (layer F.Cu) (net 14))
 (segment (start 135.89 104.14) (end 132.08 100.33) (width 0.25) (layer B.Cu) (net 40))
 (segment (start 135.89 105.41) (end 135.89 104.14) (width 0.25) (layer B.Cu) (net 40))
 (segment (start 157.48 66.04) (end 130.81 66.04) (width 0.25) (layer F.Cu) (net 16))
 (segment (start 130.81 66.04) (end 129.54 64.77) (width 0.25) (layer F.Cu) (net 16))
 (segment (start 129.54 64.77) (end 129.54 59.69) (width 0.25) (layer F.Cu) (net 16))
 (segment (start 132.08 91.44) (end 130.81 91.44) (width 0.25) (layer B.Cu) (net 16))
 (segment (start 130.81 91.44) (end 128.27 88.9) (width 0.25) (layer B.Cu) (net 16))
 (segment (start 128.27 88.9) (end 128.27 84.651839) (width 0.25) (layer B.Cu) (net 16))
 (segment (start 128.27 84.651839) (end 128.27 80.01) (width 0.25) (layer B.Cu) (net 16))
 (segment (start 128.27 80.01) (end 124.46 80.01) (width 0.25) (layer B.Cu) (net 16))
 (via (at 118.11 73.66) (size 0.8) (drill 0.4) (layers F.Cu B.Cu) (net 16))
 (segment (start 124.46 80.01) (end 118.11 73.66) (width 0.25) (layer B.Cu) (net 16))
 (segment (start 118.11 73.66) (end 127 64.77) (width 0.25) (layer F.Cu) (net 16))
 (segment (start 127 64.77) (end 129.54 64.77) (width 0.25) (layer F.Cu) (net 16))
 (segment (start 139.7 100.33) (end 139.7 92.71) (width 0.25) (layer B.Cu) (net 13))
 (segment (start 139.7 92.71) (end 135.89 88.9) (width 0.25) (layer B.Cu) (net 13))
 (segment (start 135.89 88.9) (end 133.35 88.9) (width 0.25) (layer B.Cu) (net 13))
 (segment (start 132.08 87.63) (end 132.08 85.09) (width 0.25) (layer B.Cu) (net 13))
 (segment (start 133.35 88.9) (end 132.08 87.63) (width 0.25) (layer B.Cu) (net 13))
 (segment (start 154.94 92.71) (end 152.4 92.71) (width 0.25) (layer F.Cu) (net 28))
 (segment (start 152.4 92.71) (end 152.4 83.82) (width 0.25) (layer F.Cu) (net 28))
 (segment (start 152.4 83.82) (end 153.67 82.55) (width 0.25) (layer F.Cu) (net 28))
 (segment (start 153.67 82.55) (end 154.94 82.55) (width 0.25) (layer F.Cu) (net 28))
 (segment (start 111.76 83.84) (end 111.76 85.09) (width 0.25) (layer F.Cu) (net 28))
 (segment (start 113.05 82.55) (end 111.76 83.84) (width 0.25) (layer F.Cu) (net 28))
 (segment (start 154.94 82.55) (end 113.05 82.55) (width 0.25) (layer F.Cu) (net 28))
 (segment (start 110.49 91.44) (end 110.49 90.17) (width 0.25) (layer B.Cu) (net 12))
 (segment (start 110.49 90.17) (end 107.95 87.63) (width 0.25) (layer B.Cu) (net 12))
 (segment (start 107.95 87.63) (end 102.431839 87.63) (width 0.25) (layer B.Cu) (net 12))
 (segment (start 102.431839 87.63) (end 99.06 87.63) (width 0.25) (layer B.Cu) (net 12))
 (segment (start 99.06 87.63) (end 99.06 82.55) (width 0.25) (layer B.Cu) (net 12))
 (segment (start 99.06 82.55) (end 109.22 72.39) (width 0.25) (layer B.Cu) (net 12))
 (segment (start 109.22 72.39) (end 110.49 71.12) (width 0.25) (layer B.Cu) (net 12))
 (via (at 116.84 71.12) (size 0.8) (drill 0.4) (layers F.Cu B.Cu) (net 12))
 (segment (start 110.49 71.12) (end 116.84 71.12) (width 0.25) (layer B.Cu) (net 12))
 (via (at 124.46 63.5) (size 0.8) (drill 0.4) (layers F.Cu B.Cu) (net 12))
 (segment (start 134.62 63.5) (end 134.62 59.69) (width 0.25) (layer B.Cu) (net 12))
 (segment (start 116.84 71.12) (end 124.46 63.5) (width 0.25) (layer F.Cu) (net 12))
 (segment (start 124.46 63.5) (end 134.62 63.5) (width 0.25) (layer B.Cu) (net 12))
 (segment (start 137.16 85.09) (end 137.16 81.28) (width 0.25) (layer B.Cu) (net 9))
 (segment (start 137.16 81.28) (end 138.43 80.01) (width 0.25) (layer B.Cu) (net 9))
 (segment (start 138.43 80.01) (end 149.86 80.01) (width 0.25) (layer B.Cu) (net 9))
 (segment (start 149.86 80.01) (end 151.13 81.28) (width 0.25) (layer B.Cu) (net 9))
 (segment (start 151.13 81.28) (end 151.13 86.36) (width 0.25) (layer B.Cu) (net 9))
 (segment (start 152.4 87.63) (end 154.94 87.63) (width 0.25) (layer B.Cu) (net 9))
 (segment (start 151.13 86.36) (end 152.4 87.63) (width 0.25) (layer B.Cu) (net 9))
 (segment (start 167.64 85.09) (end 171.45 88.9) (width 0.25) (layer B.Cu) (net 9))
 (segment (start 154.94 87.63) (end 157.48 85.09) (width 0.25) (layer B.Cu) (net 9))
 (segment (start 157.48 85.09) (end 167.64 85.09) (width 0.25) (layer B.Cu) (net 9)))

